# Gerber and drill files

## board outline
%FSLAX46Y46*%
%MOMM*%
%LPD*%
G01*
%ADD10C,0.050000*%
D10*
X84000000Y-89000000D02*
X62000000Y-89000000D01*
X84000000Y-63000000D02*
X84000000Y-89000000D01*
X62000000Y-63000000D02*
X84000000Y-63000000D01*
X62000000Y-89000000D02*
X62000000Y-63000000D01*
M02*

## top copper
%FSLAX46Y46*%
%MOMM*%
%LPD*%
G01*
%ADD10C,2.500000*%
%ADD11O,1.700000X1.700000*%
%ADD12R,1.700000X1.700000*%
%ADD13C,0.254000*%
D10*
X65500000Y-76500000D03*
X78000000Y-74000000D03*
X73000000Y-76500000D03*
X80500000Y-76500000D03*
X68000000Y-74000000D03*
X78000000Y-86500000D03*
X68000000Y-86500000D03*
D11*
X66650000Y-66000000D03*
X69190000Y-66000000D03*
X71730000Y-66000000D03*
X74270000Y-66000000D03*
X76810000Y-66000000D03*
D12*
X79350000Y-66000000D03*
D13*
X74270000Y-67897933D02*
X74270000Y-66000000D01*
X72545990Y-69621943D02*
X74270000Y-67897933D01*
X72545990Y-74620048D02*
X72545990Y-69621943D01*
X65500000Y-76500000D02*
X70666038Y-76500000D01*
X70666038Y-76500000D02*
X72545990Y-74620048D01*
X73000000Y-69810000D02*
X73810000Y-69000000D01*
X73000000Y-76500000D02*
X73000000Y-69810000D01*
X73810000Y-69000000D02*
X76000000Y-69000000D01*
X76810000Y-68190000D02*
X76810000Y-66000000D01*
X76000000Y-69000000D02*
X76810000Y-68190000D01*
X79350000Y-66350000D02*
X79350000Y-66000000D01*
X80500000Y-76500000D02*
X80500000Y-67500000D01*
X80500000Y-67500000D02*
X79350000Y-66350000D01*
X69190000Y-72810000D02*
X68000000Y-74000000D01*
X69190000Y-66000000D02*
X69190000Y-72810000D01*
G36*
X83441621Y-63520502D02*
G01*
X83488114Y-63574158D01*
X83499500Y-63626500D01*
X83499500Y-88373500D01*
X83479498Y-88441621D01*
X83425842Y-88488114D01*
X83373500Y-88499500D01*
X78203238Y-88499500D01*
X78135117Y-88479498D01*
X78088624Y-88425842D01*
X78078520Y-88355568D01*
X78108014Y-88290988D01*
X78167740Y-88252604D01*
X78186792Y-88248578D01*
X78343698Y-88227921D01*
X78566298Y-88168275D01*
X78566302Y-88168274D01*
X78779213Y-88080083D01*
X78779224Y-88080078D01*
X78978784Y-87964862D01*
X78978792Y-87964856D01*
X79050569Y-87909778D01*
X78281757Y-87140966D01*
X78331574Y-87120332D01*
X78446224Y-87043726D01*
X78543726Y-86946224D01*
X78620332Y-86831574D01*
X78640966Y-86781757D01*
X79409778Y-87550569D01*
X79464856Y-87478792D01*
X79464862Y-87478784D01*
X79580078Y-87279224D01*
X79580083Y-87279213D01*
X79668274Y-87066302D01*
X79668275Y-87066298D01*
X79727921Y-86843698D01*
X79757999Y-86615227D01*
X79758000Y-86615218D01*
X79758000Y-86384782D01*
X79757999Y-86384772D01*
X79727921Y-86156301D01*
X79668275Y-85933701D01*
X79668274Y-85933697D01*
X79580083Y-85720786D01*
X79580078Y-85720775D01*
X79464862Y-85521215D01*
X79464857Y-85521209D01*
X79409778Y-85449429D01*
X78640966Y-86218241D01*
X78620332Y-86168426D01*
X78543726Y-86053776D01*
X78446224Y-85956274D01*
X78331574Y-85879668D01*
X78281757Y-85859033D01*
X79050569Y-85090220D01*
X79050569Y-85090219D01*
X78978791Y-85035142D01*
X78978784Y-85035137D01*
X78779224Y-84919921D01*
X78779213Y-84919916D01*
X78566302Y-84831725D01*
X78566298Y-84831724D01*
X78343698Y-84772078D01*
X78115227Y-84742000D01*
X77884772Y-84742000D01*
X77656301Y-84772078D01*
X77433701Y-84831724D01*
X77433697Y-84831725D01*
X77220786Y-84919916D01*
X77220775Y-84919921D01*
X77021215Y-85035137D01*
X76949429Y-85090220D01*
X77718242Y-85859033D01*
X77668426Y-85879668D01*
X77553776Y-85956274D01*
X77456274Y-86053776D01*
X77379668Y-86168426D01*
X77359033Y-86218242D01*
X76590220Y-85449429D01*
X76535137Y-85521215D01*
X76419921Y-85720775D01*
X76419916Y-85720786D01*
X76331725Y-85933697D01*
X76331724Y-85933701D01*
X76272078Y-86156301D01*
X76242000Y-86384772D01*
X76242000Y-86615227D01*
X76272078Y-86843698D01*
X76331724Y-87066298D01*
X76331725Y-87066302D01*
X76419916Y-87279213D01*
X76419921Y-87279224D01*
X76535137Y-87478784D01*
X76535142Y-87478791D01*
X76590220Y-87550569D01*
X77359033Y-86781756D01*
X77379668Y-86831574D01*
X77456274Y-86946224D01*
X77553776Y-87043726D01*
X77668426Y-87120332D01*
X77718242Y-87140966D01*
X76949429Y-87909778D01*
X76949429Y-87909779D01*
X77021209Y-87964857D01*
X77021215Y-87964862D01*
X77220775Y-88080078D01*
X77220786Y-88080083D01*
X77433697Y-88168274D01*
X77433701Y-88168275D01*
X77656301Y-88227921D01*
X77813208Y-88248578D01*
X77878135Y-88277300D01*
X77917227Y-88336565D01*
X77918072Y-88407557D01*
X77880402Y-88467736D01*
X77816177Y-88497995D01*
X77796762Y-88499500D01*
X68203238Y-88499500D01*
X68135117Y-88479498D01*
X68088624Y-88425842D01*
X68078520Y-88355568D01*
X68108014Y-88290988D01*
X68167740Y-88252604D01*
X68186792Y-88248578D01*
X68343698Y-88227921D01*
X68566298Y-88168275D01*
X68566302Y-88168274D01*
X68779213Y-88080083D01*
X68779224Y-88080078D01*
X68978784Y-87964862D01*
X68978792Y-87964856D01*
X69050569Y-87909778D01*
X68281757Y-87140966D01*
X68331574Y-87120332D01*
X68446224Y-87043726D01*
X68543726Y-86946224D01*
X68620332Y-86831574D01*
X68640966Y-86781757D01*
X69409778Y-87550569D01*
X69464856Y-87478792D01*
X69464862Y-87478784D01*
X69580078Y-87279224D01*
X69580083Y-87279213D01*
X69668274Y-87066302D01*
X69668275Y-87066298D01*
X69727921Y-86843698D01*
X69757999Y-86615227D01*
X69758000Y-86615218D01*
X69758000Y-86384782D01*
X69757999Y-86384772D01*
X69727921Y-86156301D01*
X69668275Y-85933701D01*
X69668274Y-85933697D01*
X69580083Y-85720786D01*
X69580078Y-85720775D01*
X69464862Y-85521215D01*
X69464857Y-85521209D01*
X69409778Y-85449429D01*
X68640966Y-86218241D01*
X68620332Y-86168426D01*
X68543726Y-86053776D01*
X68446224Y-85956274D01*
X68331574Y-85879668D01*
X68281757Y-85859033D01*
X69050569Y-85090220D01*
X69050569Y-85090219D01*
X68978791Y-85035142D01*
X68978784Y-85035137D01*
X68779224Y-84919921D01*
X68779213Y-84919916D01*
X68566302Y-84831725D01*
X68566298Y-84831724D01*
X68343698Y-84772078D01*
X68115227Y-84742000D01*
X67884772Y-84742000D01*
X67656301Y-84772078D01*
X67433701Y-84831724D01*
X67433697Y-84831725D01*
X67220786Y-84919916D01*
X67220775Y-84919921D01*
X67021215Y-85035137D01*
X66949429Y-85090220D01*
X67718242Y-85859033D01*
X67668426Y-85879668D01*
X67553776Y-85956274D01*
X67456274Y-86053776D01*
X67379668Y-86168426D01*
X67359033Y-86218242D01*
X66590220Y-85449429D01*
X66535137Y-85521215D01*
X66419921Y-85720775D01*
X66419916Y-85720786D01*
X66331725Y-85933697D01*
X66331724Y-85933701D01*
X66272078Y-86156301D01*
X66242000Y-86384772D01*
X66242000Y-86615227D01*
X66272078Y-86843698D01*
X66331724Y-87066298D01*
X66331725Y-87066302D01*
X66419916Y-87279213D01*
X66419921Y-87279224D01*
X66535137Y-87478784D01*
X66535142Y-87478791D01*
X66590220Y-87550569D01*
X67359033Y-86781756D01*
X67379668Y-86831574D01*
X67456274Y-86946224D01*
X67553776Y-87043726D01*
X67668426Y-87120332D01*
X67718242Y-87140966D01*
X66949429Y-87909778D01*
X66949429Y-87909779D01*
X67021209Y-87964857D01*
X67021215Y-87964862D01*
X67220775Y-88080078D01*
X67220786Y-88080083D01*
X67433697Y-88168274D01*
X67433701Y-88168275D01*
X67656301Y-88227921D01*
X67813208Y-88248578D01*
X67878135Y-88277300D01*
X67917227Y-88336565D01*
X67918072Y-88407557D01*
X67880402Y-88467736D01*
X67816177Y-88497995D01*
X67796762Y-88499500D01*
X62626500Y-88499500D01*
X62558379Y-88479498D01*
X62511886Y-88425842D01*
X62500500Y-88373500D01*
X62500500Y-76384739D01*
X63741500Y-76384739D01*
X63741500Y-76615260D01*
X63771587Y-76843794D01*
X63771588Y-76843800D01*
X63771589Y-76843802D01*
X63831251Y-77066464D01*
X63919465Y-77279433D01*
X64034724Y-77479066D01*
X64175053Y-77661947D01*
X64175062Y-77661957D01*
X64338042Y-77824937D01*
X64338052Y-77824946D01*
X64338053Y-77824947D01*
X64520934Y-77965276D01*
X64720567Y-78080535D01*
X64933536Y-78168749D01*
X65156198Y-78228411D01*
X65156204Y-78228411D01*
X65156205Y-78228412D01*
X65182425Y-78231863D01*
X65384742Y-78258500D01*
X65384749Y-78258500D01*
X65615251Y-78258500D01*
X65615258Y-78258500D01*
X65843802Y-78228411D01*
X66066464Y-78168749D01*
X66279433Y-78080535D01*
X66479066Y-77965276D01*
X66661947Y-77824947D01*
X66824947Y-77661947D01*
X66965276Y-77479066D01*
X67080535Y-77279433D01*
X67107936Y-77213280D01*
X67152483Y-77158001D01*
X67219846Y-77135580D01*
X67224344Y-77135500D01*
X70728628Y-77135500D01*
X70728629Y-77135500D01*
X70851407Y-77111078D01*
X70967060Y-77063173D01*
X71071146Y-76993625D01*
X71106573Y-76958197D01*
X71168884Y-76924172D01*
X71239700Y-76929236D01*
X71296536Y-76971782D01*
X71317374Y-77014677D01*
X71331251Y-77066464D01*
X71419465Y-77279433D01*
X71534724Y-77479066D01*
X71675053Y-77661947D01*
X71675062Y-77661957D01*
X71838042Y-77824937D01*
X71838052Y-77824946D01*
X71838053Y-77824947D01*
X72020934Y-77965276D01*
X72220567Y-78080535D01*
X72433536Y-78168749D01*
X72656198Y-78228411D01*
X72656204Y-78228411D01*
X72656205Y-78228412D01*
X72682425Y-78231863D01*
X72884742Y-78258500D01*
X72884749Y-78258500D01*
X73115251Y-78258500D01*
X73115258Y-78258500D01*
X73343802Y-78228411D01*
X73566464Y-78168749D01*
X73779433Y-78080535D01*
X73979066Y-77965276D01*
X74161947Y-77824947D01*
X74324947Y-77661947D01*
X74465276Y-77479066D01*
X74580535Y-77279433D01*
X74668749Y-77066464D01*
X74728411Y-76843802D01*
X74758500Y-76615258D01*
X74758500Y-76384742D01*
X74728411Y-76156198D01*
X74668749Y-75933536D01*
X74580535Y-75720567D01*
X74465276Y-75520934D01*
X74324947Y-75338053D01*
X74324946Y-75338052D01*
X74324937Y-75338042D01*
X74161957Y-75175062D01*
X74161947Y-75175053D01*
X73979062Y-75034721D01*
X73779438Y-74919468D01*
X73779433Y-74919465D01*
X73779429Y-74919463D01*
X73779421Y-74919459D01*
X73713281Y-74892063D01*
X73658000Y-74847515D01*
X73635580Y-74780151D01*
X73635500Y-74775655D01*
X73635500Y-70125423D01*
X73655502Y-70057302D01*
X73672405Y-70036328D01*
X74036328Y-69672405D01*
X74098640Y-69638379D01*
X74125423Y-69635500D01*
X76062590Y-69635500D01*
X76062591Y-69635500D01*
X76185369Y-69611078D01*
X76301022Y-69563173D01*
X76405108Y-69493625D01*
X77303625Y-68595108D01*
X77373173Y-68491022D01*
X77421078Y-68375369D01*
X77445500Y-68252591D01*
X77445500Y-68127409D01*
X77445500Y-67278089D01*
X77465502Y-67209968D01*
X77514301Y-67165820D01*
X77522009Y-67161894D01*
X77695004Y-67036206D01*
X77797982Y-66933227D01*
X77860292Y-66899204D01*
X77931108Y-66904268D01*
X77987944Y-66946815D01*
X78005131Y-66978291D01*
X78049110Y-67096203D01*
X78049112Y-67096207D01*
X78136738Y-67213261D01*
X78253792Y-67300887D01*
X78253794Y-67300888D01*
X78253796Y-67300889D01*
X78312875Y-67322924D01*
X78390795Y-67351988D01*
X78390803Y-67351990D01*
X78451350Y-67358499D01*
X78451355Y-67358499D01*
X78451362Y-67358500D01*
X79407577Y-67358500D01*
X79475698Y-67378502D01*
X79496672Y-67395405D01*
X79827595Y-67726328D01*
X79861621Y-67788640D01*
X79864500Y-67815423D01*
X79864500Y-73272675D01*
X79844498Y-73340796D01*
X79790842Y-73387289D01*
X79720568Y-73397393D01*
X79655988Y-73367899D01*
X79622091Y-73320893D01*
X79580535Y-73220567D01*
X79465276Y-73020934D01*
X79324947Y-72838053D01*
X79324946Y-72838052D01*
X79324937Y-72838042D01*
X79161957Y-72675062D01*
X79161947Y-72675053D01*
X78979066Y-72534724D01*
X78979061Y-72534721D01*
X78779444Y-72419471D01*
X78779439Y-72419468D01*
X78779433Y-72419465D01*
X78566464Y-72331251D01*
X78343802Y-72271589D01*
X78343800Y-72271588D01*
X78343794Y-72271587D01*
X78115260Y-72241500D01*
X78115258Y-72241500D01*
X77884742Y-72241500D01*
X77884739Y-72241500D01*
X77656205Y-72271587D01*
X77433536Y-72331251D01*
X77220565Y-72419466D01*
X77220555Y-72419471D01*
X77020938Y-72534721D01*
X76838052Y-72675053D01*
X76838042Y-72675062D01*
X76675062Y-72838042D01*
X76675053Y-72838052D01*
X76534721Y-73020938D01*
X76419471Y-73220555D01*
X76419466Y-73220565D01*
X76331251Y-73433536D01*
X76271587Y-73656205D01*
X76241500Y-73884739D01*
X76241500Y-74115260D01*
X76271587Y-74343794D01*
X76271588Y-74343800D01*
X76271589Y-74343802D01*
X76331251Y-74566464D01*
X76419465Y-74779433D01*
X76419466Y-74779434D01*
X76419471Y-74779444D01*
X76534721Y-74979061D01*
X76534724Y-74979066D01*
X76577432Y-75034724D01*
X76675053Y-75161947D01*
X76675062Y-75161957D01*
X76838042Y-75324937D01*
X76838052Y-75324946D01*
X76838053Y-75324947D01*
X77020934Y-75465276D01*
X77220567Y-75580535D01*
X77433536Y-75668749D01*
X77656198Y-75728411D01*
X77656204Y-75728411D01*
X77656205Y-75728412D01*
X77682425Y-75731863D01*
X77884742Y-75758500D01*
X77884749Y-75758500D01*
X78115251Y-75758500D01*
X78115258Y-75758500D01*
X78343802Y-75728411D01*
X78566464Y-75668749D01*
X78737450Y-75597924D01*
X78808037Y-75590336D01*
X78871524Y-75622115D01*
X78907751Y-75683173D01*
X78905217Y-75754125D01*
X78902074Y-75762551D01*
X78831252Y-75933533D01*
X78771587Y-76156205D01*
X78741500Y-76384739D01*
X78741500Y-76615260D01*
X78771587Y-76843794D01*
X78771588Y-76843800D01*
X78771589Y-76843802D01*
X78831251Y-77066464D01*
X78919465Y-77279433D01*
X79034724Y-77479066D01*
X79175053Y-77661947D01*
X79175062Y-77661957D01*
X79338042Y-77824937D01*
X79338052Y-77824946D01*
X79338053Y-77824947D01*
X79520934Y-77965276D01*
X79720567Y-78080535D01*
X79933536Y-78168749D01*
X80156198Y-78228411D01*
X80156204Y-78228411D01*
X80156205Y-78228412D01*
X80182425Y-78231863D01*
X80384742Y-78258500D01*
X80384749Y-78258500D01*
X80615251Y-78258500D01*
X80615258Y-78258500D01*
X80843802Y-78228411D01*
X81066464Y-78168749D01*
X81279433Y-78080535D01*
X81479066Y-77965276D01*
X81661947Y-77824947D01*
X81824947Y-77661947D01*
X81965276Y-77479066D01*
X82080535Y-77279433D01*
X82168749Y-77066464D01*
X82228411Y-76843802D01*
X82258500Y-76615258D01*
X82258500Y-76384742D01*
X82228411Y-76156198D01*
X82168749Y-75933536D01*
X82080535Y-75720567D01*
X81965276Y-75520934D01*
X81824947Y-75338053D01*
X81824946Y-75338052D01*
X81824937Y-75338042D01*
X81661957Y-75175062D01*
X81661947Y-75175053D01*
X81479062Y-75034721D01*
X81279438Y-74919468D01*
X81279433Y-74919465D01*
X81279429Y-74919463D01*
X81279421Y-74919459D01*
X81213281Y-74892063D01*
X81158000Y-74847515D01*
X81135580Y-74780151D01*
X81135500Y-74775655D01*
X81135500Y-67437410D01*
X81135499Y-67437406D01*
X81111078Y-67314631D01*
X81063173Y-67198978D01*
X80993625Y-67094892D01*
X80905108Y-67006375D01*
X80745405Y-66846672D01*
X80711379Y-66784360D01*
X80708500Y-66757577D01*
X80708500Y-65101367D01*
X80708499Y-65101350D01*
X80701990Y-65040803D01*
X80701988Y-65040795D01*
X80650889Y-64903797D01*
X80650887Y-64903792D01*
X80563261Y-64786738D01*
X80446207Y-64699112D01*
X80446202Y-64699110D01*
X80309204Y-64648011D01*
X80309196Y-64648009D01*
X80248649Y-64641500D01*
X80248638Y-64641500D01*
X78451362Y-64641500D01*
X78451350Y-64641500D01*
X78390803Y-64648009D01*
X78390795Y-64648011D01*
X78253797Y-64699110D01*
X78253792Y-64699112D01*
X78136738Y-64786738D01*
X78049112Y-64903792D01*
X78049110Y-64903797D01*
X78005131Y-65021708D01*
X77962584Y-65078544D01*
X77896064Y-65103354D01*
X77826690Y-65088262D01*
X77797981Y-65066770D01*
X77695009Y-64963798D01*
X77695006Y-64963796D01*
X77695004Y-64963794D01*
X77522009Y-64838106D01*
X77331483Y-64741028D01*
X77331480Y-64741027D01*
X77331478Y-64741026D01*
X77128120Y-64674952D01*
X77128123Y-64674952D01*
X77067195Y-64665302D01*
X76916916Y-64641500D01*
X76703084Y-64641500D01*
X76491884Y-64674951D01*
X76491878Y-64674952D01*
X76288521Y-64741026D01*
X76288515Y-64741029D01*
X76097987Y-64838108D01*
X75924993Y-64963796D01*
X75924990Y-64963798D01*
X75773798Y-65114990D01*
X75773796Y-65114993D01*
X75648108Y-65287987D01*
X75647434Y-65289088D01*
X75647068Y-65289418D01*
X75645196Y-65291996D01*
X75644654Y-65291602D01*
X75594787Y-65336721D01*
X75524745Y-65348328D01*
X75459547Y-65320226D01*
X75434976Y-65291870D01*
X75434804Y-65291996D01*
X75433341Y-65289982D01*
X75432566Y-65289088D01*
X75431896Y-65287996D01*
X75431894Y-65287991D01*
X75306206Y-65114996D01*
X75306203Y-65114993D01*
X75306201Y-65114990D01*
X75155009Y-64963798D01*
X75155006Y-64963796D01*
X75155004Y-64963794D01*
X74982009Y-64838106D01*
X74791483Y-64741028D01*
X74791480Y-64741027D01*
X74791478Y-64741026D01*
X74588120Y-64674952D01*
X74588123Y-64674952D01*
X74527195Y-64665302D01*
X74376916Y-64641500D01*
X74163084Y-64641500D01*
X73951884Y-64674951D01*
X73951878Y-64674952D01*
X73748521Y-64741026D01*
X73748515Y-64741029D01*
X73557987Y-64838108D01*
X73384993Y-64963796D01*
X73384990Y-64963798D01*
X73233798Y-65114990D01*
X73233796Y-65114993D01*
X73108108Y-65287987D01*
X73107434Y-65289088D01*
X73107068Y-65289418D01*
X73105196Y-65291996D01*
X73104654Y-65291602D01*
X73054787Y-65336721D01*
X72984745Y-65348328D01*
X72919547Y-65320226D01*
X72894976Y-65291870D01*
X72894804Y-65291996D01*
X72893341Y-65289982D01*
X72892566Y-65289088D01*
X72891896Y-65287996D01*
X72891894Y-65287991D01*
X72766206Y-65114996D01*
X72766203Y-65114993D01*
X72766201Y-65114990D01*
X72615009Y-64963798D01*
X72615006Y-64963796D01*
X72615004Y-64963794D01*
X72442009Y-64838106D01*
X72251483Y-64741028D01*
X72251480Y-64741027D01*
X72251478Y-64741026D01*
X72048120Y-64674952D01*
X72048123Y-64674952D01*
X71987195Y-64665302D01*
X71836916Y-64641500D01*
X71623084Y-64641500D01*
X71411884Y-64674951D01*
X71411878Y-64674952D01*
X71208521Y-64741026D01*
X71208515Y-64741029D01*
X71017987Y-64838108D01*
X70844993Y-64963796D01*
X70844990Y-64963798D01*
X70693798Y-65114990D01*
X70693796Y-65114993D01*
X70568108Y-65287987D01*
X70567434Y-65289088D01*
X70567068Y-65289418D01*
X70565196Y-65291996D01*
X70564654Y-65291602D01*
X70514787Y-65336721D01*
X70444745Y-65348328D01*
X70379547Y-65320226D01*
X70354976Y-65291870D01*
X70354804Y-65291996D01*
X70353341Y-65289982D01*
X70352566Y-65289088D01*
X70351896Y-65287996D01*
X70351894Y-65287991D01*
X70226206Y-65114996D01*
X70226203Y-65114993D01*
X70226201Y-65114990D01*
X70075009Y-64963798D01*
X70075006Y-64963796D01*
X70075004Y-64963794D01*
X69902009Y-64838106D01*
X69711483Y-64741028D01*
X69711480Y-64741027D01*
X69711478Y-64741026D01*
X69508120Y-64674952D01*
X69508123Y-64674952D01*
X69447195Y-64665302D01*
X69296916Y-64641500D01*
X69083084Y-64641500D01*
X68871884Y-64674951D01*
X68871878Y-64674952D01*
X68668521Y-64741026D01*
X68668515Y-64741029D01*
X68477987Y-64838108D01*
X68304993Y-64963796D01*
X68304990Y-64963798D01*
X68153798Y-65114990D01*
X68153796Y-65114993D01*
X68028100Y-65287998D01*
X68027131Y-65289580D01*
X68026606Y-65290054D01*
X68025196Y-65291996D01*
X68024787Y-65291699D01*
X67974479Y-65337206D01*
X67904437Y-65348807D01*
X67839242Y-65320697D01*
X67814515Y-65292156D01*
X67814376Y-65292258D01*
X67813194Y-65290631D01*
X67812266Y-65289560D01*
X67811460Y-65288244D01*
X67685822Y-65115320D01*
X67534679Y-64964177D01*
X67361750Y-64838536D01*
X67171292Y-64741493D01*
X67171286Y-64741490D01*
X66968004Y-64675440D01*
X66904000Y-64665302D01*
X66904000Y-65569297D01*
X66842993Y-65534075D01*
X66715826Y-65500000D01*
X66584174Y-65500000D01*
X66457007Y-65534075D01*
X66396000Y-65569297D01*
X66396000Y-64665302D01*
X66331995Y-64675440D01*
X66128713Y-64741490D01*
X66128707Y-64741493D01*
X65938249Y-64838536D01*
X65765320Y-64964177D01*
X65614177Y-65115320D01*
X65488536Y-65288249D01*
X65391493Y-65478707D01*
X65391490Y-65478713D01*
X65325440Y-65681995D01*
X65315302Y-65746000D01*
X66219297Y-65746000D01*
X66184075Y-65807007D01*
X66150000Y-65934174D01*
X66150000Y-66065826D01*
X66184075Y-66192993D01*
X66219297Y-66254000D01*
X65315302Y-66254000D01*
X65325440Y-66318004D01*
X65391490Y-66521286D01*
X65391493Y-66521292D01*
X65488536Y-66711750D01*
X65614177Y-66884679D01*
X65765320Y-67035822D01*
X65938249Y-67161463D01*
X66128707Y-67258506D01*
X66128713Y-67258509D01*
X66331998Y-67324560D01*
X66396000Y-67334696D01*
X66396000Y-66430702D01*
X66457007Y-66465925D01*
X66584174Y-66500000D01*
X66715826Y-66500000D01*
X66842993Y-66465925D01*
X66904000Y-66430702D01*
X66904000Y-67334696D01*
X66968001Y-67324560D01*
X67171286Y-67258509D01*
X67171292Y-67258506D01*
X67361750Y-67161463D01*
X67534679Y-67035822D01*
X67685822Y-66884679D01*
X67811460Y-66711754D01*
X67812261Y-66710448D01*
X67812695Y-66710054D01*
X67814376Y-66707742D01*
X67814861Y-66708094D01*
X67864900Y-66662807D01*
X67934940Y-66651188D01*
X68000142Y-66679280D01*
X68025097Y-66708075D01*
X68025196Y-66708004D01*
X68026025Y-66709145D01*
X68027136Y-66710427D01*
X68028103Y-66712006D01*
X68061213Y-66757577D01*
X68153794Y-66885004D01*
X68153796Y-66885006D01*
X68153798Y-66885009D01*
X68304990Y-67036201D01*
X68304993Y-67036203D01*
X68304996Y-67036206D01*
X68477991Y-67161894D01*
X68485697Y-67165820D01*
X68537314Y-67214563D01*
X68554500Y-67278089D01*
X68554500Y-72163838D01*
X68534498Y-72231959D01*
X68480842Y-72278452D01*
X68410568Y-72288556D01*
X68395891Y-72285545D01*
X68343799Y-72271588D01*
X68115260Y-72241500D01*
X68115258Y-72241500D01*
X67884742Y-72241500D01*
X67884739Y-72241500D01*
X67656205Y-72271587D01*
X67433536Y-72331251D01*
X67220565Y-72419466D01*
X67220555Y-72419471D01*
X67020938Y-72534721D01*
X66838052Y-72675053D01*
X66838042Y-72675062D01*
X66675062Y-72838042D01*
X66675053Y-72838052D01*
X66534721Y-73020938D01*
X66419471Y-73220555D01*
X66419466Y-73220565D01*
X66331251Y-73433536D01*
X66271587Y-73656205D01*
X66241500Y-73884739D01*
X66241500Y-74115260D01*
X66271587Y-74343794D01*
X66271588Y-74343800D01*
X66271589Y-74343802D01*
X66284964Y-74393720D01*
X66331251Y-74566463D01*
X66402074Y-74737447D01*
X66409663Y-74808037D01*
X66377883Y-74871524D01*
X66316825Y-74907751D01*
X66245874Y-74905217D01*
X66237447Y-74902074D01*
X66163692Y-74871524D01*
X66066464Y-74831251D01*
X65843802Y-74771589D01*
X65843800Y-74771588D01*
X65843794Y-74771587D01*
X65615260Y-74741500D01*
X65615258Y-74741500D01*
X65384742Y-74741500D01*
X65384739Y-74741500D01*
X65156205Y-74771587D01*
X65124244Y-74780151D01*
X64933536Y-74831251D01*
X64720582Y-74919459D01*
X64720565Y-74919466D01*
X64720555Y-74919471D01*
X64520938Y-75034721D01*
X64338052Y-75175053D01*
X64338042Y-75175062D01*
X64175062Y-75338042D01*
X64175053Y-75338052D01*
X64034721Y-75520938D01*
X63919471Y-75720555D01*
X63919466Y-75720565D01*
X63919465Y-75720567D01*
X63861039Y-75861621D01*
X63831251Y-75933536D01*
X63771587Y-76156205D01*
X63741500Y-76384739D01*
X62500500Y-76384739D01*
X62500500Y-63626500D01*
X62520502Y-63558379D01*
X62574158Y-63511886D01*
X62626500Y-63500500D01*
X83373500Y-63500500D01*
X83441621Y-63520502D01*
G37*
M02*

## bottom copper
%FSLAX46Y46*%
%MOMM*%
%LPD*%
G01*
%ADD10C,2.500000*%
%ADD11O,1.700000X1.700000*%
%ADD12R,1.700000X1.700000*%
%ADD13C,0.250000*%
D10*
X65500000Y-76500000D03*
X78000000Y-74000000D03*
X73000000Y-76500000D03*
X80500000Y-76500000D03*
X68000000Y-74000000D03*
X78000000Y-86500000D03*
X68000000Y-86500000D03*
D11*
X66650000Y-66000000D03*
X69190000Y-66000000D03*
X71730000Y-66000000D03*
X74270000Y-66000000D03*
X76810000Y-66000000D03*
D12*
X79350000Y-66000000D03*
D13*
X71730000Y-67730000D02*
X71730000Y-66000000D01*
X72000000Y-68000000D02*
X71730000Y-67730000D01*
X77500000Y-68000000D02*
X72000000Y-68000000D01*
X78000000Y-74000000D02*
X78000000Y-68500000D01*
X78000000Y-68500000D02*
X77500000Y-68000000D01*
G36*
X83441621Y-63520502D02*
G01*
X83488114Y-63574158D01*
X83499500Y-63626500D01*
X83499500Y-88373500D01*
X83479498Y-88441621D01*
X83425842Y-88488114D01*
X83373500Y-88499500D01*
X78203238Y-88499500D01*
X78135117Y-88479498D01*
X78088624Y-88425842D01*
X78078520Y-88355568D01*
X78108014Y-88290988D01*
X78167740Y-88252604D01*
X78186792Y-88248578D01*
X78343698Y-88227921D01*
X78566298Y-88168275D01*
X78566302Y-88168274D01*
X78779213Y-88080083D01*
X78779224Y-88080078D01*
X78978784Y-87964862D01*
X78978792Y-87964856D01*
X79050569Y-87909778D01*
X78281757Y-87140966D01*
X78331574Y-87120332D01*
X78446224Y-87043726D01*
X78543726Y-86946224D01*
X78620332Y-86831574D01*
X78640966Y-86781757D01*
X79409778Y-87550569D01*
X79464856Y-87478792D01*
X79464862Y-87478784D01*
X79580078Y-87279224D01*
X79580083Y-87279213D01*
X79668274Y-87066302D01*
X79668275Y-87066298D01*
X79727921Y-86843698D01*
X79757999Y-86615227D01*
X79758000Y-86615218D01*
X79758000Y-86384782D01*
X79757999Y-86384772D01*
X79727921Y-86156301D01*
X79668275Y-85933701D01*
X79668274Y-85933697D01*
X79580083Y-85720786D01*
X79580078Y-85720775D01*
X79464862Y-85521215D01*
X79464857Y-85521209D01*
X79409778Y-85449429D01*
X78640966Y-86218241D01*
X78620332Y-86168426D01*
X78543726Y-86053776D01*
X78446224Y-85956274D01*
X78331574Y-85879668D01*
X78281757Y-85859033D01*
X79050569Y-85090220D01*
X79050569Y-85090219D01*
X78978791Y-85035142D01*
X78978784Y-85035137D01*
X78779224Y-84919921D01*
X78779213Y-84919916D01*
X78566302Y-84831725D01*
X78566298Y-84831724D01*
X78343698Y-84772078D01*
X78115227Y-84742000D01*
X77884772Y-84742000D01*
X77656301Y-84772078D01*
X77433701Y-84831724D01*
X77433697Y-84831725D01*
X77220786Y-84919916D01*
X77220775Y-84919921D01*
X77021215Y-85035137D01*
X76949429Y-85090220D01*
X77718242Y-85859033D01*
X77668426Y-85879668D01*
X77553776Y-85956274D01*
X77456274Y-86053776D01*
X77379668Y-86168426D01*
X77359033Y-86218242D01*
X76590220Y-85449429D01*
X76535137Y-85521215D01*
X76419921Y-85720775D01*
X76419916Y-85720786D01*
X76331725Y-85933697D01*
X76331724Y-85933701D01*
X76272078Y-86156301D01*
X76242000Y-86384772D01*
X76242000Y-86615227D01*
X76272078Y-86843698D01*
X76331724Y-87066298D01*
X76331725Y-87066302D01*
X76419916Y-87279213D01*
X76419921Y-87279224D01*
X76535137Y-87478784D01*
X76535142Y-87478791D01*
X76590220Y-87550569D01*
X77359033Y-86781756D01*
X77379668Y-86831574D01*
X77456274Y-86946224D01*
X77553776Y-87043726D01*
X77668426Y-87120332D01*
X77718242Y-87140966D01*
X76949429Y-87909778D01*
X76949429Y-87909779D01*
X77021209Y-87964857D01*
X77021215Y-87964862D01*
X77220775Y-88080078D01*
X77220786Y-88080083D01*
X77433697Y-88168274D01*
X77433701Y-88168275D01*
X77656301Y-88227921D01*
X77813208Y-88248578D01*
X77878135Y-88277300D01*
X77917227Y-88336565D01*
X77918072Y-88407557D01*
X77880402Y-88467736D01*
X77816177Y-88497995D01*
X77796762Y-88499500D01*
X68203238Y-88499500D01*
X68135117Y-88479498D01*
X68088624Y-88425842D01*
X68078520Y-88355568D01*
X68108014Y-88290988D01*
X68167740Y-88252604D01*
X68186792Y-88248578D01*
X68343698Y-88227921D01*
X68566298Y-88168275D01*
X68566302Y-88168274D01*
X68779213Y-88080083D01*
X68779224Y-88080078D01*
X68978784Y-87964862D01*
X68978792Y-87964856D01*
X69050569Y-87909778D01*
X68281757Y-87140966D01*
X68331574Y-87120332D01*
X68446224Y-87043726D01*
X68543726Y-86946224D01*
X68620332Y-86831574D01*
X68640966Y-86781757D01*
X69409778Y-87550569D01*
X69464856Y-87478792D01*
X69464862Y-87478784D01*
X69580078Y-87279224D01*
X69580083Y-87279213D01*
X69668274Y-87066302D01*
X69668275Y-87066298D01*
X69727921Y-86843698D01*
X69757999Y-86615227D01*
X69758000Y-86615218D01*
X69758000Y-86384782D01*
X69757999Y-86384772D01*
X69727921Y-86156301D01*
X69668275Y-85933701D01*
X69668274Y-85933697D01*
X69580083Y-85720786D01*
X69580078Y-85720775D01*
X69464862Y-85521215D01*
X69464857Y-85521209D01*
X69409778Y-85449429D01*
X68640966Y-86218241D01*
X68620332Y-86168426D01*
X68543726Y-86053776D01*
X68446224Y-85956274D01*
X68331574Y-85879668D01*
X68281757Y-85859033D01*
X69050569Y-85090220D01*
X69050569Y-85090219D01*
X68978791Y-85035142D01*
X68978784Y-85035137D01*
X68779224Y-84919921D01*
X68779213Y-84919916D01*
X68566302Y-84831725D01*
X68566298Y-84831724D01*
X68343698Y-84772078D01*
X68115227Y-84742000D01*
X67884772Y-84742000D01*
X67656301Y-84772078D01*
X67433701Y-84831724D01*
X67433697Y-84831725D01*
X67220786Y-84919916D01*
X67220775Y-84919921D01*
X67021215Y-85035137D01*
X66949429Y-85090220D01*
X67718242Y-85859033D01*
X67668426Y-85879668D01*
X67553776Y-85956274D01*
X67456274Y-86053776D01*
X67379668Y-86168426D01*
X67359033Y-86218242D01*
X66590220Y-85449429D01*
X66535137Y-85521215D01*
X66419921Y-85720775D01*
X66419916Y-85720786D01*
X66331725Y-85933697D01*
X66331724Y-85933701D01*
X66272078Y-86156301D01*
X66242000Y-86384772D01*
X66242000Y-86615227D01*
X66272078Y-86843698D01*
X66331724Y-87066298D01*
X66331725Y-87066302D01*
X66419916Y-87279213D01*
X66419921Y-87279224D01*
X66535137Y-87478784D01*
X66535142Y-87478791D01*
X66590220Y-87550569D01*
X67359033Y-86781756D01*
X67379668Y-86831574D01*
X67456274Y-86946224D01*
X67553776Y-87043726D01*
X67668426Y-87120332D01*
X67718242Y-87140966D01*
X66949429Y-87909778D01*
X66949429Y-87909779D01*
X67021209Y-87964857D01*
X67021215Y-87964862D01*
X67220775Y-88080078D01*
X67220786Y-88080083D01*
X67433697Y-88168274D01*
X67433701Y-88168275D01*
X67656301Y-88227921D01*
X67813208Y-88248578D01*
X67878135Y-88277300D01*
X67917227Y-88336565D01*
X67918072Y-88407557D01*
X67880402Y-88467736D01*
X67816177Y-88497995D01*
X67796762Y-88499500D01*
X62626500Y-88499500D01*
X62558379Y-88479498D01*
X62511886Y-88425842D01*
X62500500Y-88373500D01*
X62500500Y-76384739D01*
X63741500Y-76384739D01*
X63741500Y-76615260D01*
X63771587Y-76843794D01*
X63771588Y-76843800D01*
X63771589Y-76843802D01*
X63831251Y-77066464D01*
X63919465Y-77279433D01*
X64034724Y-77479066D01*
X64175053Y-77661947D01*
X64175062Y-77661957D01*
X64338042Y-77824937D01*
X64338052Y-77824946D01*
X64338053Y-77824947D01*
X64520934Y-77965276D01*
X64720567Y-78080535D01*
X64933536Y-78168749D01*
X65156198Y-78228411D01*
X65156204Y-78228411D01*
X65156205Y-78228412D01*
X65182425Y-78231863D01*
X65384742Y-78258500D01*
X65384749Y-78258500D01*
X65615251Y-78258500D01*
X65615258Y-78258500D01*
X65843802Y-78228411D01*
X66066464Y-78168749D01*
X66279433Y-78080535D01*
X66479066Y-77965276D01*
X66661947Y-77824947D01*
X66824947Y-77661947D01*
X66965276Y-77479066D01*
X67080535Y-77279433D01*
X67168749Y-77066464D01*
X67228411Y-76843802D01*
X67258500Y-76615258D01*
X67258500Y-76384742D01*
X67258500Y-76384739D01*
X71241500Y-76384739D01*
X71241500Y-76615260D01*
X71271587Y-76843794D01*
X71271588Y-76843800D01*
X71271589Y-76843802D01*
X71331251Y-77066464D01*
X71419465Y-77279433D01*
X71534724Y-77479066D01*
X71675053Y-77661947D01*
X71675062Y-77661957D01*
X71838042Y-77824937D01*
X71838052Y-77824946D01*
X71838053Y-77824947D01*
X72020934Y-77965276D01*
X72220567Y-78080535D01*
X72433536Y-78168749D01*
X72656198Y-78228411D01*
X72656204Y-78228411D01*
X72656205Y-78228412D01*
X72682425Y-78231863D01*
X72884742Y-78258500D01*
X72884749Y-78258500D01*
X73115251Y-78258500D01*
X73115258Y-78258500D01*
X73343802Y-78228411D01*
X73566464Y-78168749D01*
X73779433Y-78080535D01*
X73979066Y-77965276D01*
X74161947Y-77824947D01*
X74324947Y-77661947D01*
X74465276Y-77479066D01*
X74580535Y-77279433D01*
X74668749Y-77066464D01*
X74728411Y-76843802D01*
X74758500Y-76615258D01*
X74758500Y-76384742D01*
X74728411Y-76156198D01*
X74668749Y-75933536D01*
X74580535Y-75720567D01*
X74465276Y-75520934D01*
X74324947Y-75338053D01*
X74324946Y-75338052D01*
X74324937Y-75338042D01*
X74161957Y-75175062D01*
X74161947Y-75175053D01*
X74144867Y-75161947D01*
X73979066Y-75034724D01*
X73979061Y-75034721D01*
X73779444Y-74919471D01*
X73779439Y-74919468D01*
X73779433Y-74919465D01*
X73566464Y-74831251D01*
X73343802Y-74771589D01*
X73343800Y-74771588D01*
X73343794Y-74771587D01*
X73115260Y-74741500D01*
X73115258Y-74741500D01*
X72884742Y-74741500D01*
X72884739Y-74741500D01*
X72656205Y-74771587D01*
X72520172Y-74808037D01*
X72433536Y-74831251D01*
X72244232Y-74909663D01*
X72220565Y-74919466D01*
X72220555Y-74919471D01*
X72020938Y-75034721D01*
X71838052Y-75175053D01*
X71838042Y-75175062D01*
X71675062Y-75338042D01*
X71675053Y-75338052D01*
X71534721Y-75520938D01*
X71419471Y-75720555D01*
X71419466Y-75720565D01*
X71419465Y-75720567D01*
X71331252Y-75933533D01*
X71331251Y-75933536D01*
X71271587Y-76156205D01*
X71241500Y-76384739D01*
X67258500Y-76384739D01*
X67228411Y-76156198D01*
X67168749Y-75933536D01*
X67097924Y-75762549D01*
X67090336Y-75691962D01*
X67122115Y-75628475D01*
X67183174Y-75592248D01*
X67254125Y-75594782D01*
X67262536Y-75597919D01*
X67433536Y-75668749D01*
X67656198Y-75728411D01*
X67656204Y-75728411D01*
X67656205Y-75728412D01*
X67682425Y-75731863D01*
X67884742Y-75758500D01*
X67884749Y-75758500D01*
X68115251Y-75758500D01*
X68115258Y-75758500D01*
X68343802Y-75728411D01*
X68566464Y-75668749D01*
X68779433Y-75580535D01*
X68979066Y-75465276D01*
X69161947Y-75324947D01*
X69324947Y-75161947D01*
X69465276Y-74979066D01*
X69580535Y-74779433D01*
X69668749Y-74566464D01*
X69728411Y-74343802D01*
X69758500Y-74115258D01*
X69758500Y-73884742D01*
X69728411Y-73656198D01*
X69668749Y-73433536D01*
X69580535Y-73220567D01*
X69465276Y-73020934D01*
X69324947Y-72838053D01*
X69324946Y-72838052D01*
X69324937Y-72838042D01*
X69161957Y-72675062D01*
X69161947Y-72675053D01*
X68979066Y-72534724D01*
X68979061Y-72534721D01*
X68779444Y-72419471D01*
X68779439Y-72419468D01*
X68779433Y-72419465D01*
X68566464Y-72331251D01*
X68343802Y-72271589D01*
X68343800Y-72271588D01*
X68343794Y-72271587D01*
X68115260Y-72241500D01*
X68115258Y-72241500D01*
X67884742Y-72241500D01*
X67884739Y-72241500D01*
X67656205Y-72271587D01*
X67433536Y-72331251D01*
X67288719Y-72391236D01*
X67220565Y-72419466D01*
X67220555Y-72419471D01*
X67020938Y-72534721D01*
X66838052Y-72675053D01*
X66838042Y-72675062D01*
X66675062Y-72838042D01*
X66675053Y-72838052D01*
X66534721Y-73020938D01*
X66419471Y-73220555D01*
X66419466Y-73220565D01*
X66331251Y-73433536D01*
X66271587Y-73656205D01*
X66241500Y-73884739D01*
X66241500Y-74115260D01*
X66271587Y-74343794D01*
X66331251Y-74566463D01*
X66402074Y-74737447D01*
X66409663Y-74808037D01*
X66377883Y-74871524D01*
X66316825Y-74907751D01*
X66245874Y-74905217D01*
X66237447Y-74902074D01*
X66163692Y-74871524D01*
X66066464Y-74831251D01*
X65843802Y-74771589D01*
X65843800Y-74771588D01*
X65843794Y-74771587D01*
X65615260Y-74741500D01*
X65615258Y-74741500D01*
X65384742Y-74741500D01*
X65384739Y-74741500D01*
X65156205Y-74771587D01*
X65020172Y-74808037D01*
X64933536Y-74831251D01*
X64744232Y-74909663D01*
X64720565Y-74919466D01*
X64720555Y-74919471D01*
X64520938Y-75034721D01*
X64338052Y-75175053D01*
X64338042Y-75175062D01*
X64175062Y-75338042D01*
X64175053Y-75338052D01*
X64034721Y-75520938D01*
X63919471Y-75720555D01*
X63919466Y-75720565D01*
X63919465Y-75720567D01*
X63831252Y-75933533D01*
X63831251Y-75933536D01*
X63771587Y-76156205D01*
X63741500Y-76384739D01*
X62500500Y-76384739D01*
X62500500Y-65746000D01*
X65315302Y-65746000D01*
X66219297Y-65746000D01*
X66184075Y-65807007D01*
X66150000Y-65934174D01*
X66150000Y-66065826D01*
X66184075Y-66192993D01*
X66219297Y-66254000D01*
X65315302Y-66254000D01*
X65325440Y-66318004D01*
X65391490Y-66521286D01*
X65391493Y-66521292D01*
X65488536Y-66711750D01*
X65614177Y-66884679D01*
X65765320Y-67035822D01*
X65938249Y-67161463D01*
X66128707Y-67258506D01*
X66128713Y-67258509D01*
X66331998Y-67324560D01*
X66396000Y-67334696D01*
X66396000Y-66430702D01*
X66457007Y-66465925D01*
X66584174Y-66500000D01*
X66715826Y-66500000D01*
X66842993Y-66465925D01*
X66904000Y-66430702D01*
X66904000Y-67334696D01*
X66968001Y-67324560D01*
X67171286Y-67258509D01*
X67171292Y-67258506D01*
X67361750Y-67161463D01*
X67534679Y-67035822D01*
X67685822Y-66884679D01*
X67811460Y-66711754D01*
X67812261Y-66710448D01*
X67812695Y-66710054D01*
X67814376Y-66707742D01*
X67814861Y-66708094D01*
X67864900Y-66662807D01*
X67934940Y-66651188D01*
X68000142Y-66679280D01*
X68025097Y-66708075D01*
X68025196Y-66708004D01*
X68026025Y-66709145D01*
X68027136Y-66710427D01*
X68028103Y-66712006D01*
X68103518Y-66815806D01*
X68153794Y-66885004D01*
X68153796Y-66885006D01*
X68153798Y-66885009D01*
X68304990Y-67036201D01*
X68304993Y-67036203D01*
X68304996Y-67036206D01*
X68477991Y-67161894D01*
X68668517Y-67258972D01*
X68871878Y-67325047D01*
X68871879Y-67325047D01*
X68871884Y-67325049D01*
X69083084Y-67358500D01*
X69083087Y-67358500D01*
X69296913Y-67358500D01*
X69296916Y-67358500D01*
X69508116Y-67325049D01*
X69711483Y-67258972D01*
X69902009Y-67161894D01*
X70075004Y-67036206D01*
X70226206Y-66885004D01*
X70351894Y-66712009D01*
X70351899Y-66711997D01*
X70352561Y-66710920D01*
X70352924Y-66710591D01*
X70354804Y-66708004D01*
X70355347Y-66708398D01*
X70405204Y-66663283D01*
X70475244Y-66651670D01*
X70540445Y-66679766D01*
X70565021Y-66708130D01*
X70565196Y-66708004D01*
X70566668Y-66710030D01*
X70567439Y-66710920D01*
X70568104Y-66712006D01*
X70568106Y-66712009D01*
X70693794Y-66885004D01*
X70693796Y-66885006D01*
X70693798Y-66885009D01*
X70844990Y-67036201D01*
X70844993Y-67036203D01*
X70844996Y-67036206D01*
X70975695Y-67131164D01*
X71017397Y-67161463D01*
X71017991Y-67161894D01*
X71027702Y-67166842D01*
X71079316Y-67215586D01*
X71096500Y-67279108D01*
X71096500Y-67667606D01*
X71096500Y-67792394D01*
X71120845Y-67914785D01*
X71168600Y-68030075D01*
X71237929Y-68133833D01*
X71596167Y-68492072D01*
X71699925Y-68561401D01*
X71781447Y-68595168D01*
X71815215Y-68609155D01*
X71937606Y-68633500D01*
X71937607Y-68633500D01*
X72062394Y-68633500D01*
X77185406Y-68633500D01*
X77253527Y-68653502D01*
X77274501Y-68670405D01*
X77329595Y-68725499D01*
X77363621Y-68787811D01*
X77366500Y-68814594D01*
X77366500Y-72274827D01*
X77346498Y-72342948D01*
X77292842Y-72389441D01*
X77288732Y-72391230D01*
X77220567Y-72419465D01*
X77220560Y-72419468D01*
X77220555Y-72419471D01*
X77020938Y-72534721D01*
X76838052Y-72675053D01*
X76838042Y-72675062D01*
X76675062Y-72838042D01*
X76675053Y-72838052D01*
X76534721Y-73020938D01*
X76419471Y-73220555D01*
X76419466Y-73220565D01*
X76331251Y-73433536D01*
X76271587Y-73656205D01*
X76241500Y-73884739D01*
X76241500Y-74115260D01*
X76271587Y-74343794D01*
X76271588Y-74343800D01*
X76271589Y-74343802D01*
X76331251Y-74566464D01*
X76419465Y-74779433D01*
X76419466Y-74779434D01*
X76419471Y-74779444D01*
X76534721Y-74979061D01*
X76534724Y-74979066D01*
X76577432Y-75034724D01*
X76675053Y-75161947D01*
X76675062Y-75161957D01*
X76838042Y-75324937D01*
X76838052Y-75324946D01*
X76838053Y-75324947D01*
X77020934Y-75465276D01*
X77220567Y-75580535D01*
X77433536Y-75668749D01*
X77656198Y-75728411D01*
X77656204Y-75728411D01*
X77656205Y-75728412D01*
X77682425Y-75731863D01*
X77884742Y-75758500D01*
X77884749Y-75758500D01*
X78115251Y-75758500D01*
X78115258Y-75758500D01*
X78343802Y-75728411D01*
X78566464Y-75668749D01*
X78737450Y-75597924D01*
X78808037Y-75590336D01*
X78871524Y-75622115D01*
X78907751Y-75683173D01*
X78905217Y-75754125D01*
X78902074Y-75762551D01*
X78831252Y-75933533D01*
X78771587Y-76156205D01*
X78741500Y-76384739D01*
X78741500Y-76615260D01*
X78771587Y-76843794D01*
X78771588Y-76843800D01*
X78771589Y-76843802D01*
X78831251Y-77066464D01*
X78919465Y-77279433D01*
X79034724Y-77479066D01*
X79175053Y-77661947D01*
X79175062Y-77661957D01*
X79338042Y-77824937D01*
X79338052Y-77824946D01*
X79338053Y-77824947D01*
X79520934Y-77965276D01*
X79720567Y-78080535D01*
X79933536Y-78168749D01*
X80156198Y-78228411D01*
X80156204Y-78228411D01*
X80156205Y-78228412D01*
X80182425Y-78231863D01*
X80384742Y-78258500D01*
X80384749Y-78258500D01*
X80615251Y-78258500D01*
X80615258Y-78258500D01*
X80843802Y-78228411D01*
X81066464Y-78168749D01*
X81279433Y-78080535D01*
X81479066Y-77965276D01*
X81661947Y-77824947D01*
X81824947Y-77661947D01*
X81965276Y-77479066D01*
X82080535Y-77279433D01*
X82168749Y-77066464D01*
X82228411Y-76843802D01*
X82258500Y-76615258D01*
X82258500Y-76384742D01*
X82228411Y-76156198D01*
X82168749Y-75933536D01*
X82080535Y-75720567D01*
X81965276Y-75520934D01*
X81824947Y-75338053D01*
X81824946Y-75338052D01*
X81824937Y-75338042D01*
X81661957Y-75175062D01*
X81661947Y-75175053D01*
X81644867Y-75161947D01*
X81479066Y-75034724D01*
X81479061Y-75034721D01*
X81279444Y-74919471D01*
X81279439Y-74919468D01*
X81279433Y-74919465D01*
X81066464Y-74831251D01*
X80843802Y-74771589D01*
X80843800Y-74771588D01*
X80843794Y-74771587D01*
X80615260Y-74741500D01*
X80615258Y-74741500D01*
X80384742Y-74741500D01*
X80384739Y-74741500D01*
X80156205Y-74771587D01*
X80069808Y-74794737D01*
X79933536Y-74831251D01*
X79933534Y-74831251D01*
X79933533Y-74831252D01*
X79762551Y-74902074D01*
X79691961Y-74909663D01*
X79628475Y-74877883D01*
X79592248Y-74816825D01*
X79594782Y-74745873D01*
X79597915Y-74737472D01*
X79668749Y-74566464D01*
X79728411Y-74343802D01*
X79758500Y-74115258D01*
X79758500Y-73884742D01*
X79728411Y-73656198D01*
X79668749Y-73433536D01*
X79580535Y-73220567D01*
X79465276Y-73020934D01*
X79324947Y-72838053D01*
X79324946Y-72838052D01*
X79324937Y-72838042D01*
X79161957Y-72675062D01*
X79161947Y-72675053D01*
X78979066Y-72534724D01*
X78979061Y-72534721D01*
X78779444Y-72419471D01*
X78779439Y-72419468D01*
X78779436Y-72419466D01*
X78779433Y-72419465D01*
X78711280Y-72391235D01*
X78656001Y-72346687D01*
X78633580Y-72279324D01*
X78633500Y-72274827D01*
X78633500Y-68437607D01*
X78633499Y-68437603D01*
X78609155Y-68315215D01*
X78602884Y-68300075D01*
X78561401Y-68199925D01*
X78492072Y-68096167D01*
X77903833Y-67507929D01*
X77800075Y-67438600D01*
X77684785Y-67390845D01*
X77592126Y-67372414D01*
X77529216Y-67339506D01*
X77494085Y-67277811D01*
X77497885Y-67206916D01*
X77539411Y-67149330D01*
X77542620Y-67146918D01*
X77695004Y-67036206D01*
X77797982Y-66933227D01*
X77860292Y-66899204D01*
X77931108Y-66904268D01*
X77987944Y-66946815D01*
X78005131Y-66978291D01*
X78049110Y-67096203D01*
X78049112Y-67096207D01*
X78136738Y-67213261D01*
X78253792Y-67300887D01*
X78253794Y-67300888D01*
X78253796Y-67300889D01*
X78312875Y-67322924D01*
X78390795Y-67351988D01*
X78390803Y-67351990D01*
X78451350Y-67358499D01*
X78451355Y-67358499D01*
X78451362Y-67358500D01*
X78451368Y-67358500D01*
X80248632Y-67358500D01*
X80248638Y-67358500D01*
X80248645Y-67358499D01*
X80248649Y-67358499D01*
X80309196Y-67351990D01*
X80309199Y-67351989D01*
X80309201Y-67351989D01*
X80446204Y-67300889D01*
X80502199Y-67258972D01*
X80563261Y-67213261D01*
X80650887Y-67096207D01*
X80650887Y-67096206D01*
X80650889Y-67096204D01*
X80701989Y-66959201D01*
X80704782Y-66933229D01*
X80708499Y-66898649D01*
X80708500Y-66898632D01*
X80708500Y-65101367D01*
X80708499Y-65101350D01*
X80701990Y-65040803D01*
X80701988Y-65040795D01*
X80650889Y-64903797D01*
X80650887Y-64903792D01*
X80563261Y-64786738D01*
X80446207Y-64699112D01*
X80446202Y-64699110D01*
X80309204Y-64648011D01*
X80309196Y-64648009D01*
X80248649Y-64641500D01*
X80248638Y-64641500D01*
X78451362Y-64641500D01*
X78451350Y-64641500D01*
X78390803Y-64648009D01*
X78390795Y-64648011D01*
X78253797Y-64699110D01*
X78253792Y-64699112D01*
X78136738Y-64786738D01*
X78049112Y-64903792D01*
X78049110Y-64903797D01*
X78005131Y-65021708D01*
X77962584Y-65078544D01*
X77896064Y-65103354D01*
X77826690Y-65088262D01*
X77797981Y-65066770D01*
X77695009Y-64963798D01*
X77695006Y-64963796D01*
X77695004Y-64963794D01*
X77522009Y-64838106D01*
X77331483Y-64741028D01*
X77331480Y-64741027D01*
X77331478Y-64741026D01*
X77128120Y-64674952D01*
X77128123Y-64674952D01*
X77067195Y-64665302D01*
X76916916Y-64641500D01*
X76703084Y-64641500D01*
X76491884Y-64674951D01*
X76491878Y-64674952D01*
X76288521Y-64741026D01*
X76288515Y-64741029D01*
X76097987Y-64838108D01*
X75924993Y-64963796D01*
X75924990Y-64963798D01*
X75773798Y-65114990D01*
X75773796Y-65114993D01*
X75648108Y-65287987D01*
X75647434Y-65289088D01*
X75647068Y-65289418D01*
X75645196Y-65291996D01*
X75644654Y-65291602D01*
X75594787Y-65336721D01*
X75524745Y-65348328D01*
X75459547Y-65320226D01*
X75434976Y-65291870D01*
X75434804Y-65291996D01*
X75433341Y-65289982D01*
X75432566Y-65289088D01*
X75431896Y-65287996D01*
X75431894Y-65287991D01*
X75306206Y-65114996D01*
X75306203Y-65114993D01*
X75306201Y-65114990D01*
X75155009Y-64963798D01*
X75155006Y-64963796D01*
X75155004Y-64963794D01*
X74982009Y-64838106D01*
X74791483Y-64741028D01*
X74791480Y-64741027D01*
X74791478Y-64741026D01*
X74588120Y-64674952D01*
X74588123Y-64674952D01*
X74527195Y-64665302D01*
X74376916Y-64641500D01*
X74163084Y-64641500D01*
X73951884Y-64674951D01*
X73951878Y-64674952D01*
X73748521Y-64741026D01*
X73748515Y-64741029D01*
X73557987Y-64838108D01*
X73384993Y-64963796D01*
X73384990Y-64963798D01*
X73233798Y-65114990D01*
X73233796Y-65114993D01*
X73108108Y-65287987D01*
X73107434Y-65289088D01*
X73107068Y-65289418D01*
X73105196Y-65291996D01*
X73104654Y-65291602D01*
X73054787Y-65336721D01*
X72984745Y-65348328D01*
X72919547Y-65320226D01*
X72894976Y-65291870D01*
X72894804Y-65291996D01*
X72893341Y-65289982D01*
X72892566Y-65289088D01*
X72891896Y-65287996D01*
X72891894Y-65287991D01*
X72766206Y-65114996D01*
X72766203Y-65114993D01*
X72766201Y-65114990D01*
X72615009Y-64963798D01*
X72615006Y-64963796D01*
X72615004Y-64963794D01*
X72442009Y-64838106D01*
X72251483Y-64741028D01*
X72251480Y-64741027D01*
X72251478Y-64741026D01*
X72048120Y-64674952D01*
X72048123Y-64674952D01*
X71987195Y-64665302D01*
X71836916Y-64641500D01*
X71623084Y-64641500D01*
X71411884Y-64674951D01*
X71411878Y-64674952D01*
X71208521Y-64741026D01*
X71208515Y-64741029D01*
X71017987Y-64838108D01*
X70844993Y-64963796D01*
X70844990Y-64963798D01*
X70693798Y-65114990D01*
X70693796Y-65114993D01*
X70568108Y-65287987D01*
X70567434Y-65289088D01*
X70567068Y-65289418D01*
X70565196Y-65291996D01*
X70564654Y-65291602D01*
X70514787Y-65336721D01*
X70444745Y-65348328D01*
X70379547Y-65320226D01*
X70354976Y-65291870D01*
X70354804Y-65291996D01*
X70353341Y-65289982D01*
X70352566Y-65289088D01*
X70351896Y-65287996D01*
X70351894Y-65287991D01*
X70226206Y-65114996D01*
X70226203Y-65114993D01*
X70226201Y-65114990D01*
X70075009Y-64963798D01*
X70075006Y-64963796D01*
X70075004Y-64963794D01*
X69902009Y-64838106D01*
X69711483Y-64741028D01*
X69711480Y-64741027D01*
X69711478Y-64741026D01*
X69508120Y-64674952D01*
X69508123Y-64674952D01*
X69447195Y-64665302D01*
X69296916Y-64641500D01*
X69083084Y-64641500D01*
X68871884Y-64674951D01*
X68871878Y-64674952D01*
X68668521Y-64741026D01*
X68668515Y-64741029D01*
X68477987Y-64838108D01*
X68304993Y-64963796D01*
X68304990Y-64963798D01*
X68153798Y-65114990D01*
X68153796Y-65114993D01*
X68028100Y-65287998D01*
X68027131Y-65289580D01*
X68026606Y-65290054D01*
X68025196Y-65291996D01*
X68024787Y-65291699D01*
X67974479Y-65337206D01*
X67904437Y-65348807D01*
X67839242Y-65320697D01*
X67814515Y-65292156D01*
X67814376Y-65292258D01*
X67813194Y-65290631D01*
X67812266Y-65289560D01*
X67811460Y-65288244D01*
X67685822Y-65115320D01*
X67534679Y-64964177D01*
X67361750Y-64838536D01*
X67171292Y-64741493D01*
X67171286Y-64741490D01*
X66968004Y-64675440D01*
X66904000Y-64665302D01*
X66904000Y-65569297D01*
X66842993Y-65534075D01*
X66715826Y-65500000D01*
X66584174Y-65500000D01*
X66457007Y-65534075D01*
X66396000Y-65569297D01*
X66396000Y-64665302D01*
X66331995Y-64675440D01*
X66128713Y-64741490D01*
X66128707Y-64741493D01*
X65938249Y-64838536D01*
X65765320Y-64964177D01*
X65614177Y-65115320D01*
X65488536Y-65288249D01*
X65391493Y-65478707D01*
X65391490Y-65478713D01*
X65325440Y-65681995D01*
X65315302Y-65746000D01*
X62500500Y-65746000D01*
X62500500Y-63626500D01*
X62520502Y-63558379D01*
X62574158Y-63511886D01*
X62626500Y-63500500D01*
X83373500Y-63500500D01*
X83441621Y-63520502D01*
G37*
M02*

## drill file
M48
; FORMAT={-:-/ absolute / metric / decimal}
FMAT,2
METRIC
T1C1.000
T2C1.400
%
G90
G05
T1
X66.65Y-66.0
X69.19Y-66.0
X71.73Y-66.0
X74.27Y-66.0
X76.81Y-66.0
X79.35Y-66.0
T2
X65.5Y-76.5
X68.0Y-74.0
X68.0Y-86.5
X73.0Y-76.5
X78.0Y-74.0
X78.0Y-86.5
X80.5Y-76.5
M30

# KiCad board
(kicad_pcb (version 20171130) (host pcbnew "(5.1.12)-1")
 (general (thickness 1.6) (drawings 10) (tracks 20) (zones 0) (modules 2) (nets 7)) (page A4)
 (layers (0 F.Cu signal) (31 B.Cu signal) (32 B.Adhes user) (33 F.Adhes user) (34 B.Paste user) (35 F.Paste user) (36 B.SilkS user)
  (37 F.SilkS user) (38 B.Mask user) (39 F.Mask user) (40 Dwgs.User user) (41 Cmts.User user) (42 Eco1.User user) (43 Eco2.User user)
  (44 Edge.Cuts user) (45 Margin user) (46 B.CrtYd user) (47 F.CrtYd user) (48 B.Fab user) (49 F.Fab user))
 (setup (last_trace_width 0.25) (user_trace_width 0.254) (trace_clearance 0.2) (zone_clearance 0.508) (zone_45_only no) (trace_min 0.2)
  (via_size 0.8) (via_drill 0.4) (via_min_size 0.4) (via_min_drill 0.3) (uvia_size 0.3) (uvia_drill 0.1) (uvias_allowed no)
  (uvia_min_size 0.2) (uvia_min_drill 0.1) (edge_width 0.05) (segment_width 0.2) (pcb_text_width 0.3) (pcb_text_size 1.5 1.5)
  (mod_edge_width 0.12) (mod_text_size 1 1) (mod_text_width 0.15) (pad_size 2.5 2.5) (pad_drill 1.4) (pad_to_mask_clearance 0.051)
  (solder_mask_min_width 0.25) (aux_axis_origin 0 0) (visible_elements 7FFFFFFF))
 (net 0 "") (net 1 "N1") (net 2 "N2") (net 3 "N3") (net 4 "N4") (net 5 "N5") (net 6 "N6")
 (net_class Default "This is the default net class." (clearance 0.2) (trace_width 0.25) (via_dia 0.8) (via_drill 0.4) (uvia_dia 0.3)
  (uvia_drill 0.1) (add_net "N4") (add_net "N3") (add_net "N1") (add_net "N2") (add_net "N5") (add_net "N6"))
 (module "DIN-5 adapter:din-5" (layer F.Cu) (at 73 79.5)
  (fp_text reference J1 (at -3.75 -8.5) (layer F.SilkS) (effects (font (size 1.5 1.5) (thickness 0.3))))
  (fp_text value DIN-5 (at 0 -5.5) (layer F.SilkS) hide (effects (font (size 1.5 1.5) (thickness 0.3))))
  (pad 3 thru_hole circle (at -7.5 -3) (size 2.5 2.5) (drill 1.4) (layers *.Cu *.Mask) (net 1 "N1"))
  (pad 4 thru_hole circle (at 5 -5.5) (size 2.5 2.5) (drill 1.4) (layers *.Cu *.Mask) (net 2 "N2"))
  (pad 2 thru_hole circle (at 0 -3) (size 2.5 2.5) (drill 1.4) (layers *.Cu *.Mask) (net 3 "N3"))
  (pad 1 thru_hole circle (at 7.5 -3) (size 2.5 2.5) (drill 1.4) (layers *.Cu *.Mask) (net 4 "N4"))
  (pad 5 thru_hole circle (at -5 -5.5) (size 2.5 2.5) (drill 1.4) (layers *.Cu *.Mask) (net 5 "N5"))
  (pad 6 thru_hole circle (at 5 7) (size 2.5 2.5) (drill 1.4) (layers *.Cu *.Mask) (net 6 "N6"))
  (pad 6 thru_hole circle (at -5 7) (size 2.5 2.5) (drill 1.4) (layers *.Cu *.Mask) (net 6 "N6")))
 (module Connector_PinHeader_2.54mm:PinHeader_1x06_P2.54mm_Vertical (layer B.Cu) (at 79.35 66 90)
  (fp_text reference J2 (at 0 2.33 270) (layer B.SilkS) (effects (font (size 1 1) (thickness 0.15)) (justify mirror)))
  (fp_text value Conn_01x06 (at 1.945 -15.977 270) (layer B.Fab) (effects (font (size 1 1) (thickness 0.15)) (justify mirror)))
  (pad 6 thru_hole oval (at 0 -12.7 90) (size 1.7 1.7) (drill 1) (layers *.Cu *.Mask) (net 6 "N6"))
  (pad 5 thru_hole oval (at 0 -10.16 90) (size 1.7 1.7) (drill 1) (layers *.Cu *.Mask) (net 5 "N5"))
  (pad 4 thru_hole oval (at 0 -7.62 90) (size 1.7 1.7) (drill 1) (layers *.Cu *.Mask) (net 2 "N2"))
  (pad 3 thru_hole oval (at 0 -5.08 90) (size 1.7 1.7) (drill 1) (layers *.Cu *.Mask) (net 1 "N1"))
  (pad 2 thru_hole oval (at 0 -2.54 90) (size 1.7 1.7) (drill 1) (layers *.Cu *.Mask) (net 3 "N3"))
  (pad 1 thru_hole rect (at 0 0 90) (size 1.7 1.7) (drill 1) (layers *.Cu *.Mask) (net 4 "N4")))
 (gr_line (start 84 89) (end 62 89) (layer Edge.Cuts) (width 0.05))
 (gr_line (start 84 63) (end 84 89) (layer Edge.Cuts) (width 0.05))
 (gr_line (start 62 63) (end 84 63) (layer Edge.Cuts) (width 0.05))
 (gr_line (start 62 89) (end 62 63) (layer Edge.Cuts) (width 0.05))
 (segment (start 74.27 67.897933) (end 74.27 66) (width 0.254) (layer F.Cu) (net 1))
 (segment (start 72.54599 69.621943) (end 74.27 67.897933) (width 0.254) (layer F.Cu) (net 1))
 (segment (start 72.54599 74.620048) (end 72.54599 69.621943) (width 0.254) (layer F.Cu) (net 1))
 (segment (start 65.5 76.5) (end 70.666038 76.5) (width 0.254) (layer F.Cu) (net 1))
 (segment (start 70.666038 76.5) (end 72.54599 74.620048) (width 0.254) (layer F.Cu) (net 1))
 (segment (start 71.73 67.73) (end 71.73 66) (width 0.25) (layer B.Cu) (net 2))
 (segment (start 72 68) (end 71.73 67.73) (width 0.25) (layer B.Cu) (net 2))
 (segment (start 77.5 68) (end 72 68) (width 0.25) (layer B.Cu) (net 2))
 (segment (start 78 74) (end 78 68.5) (width 0.25) (layer B.Cu) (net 2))
 (segment (start 78 68.5) (end 77.5 68) (width 0.25) (layer B.Cu) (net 2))
 (segment (start 73 69.81) (end 73.81 69) (width 0.254) (layer F.Cu) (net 3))
 (segment (start 73 76.5) (end 73 69.81) (width 0.254) (layer F.Cu) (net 3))
 (segment (start 73.81 69) (end 76 69) (width 0.254) (layer F.Cu) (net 3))
 (segment (start 76.81 68.19) (end 76.81 66) (width 0.254) (layer F.Cu) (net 3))
 (segment (start 76 69) (end 76.81 68.19) (width 0.254) (layer F.Cu) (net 3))
 (segment (start 79.35 66.35) (end 79.35 66) (width 0.254) (layer F.Cu) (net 4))
 (segment (start 80.5 76.5) (end 80.5 67.5) (width 0.254) (layer F.Cu) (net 4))
 (segment (start 80.5 67.5) (end 79.35 66.35) (width 0.254) (layer F.Cu) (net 4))
 (segment (start 69.19 72.81) (end 68 74) (width 0.254) (layer F.Cu) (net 5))
 (segment (start 69.19 66) (end 69.19 72.81) (width 0.254) (layer F.Cu) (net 5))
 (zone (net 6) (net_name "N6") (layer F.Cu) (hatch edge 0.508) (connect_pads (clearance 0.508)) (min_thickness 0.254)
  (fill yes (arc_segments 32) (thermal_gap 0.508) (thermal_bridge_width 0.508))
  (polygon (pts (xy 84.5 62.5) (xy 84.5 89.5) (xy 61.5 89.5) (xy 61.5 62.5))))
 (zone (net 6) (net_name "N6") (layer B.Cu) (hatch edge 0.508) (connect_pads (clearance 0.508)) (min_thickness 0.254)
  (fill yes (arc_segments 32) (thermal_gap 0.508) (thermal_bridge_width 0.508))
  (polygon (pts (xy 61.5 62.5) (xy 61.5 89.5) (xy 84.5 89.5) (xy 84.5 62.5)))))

